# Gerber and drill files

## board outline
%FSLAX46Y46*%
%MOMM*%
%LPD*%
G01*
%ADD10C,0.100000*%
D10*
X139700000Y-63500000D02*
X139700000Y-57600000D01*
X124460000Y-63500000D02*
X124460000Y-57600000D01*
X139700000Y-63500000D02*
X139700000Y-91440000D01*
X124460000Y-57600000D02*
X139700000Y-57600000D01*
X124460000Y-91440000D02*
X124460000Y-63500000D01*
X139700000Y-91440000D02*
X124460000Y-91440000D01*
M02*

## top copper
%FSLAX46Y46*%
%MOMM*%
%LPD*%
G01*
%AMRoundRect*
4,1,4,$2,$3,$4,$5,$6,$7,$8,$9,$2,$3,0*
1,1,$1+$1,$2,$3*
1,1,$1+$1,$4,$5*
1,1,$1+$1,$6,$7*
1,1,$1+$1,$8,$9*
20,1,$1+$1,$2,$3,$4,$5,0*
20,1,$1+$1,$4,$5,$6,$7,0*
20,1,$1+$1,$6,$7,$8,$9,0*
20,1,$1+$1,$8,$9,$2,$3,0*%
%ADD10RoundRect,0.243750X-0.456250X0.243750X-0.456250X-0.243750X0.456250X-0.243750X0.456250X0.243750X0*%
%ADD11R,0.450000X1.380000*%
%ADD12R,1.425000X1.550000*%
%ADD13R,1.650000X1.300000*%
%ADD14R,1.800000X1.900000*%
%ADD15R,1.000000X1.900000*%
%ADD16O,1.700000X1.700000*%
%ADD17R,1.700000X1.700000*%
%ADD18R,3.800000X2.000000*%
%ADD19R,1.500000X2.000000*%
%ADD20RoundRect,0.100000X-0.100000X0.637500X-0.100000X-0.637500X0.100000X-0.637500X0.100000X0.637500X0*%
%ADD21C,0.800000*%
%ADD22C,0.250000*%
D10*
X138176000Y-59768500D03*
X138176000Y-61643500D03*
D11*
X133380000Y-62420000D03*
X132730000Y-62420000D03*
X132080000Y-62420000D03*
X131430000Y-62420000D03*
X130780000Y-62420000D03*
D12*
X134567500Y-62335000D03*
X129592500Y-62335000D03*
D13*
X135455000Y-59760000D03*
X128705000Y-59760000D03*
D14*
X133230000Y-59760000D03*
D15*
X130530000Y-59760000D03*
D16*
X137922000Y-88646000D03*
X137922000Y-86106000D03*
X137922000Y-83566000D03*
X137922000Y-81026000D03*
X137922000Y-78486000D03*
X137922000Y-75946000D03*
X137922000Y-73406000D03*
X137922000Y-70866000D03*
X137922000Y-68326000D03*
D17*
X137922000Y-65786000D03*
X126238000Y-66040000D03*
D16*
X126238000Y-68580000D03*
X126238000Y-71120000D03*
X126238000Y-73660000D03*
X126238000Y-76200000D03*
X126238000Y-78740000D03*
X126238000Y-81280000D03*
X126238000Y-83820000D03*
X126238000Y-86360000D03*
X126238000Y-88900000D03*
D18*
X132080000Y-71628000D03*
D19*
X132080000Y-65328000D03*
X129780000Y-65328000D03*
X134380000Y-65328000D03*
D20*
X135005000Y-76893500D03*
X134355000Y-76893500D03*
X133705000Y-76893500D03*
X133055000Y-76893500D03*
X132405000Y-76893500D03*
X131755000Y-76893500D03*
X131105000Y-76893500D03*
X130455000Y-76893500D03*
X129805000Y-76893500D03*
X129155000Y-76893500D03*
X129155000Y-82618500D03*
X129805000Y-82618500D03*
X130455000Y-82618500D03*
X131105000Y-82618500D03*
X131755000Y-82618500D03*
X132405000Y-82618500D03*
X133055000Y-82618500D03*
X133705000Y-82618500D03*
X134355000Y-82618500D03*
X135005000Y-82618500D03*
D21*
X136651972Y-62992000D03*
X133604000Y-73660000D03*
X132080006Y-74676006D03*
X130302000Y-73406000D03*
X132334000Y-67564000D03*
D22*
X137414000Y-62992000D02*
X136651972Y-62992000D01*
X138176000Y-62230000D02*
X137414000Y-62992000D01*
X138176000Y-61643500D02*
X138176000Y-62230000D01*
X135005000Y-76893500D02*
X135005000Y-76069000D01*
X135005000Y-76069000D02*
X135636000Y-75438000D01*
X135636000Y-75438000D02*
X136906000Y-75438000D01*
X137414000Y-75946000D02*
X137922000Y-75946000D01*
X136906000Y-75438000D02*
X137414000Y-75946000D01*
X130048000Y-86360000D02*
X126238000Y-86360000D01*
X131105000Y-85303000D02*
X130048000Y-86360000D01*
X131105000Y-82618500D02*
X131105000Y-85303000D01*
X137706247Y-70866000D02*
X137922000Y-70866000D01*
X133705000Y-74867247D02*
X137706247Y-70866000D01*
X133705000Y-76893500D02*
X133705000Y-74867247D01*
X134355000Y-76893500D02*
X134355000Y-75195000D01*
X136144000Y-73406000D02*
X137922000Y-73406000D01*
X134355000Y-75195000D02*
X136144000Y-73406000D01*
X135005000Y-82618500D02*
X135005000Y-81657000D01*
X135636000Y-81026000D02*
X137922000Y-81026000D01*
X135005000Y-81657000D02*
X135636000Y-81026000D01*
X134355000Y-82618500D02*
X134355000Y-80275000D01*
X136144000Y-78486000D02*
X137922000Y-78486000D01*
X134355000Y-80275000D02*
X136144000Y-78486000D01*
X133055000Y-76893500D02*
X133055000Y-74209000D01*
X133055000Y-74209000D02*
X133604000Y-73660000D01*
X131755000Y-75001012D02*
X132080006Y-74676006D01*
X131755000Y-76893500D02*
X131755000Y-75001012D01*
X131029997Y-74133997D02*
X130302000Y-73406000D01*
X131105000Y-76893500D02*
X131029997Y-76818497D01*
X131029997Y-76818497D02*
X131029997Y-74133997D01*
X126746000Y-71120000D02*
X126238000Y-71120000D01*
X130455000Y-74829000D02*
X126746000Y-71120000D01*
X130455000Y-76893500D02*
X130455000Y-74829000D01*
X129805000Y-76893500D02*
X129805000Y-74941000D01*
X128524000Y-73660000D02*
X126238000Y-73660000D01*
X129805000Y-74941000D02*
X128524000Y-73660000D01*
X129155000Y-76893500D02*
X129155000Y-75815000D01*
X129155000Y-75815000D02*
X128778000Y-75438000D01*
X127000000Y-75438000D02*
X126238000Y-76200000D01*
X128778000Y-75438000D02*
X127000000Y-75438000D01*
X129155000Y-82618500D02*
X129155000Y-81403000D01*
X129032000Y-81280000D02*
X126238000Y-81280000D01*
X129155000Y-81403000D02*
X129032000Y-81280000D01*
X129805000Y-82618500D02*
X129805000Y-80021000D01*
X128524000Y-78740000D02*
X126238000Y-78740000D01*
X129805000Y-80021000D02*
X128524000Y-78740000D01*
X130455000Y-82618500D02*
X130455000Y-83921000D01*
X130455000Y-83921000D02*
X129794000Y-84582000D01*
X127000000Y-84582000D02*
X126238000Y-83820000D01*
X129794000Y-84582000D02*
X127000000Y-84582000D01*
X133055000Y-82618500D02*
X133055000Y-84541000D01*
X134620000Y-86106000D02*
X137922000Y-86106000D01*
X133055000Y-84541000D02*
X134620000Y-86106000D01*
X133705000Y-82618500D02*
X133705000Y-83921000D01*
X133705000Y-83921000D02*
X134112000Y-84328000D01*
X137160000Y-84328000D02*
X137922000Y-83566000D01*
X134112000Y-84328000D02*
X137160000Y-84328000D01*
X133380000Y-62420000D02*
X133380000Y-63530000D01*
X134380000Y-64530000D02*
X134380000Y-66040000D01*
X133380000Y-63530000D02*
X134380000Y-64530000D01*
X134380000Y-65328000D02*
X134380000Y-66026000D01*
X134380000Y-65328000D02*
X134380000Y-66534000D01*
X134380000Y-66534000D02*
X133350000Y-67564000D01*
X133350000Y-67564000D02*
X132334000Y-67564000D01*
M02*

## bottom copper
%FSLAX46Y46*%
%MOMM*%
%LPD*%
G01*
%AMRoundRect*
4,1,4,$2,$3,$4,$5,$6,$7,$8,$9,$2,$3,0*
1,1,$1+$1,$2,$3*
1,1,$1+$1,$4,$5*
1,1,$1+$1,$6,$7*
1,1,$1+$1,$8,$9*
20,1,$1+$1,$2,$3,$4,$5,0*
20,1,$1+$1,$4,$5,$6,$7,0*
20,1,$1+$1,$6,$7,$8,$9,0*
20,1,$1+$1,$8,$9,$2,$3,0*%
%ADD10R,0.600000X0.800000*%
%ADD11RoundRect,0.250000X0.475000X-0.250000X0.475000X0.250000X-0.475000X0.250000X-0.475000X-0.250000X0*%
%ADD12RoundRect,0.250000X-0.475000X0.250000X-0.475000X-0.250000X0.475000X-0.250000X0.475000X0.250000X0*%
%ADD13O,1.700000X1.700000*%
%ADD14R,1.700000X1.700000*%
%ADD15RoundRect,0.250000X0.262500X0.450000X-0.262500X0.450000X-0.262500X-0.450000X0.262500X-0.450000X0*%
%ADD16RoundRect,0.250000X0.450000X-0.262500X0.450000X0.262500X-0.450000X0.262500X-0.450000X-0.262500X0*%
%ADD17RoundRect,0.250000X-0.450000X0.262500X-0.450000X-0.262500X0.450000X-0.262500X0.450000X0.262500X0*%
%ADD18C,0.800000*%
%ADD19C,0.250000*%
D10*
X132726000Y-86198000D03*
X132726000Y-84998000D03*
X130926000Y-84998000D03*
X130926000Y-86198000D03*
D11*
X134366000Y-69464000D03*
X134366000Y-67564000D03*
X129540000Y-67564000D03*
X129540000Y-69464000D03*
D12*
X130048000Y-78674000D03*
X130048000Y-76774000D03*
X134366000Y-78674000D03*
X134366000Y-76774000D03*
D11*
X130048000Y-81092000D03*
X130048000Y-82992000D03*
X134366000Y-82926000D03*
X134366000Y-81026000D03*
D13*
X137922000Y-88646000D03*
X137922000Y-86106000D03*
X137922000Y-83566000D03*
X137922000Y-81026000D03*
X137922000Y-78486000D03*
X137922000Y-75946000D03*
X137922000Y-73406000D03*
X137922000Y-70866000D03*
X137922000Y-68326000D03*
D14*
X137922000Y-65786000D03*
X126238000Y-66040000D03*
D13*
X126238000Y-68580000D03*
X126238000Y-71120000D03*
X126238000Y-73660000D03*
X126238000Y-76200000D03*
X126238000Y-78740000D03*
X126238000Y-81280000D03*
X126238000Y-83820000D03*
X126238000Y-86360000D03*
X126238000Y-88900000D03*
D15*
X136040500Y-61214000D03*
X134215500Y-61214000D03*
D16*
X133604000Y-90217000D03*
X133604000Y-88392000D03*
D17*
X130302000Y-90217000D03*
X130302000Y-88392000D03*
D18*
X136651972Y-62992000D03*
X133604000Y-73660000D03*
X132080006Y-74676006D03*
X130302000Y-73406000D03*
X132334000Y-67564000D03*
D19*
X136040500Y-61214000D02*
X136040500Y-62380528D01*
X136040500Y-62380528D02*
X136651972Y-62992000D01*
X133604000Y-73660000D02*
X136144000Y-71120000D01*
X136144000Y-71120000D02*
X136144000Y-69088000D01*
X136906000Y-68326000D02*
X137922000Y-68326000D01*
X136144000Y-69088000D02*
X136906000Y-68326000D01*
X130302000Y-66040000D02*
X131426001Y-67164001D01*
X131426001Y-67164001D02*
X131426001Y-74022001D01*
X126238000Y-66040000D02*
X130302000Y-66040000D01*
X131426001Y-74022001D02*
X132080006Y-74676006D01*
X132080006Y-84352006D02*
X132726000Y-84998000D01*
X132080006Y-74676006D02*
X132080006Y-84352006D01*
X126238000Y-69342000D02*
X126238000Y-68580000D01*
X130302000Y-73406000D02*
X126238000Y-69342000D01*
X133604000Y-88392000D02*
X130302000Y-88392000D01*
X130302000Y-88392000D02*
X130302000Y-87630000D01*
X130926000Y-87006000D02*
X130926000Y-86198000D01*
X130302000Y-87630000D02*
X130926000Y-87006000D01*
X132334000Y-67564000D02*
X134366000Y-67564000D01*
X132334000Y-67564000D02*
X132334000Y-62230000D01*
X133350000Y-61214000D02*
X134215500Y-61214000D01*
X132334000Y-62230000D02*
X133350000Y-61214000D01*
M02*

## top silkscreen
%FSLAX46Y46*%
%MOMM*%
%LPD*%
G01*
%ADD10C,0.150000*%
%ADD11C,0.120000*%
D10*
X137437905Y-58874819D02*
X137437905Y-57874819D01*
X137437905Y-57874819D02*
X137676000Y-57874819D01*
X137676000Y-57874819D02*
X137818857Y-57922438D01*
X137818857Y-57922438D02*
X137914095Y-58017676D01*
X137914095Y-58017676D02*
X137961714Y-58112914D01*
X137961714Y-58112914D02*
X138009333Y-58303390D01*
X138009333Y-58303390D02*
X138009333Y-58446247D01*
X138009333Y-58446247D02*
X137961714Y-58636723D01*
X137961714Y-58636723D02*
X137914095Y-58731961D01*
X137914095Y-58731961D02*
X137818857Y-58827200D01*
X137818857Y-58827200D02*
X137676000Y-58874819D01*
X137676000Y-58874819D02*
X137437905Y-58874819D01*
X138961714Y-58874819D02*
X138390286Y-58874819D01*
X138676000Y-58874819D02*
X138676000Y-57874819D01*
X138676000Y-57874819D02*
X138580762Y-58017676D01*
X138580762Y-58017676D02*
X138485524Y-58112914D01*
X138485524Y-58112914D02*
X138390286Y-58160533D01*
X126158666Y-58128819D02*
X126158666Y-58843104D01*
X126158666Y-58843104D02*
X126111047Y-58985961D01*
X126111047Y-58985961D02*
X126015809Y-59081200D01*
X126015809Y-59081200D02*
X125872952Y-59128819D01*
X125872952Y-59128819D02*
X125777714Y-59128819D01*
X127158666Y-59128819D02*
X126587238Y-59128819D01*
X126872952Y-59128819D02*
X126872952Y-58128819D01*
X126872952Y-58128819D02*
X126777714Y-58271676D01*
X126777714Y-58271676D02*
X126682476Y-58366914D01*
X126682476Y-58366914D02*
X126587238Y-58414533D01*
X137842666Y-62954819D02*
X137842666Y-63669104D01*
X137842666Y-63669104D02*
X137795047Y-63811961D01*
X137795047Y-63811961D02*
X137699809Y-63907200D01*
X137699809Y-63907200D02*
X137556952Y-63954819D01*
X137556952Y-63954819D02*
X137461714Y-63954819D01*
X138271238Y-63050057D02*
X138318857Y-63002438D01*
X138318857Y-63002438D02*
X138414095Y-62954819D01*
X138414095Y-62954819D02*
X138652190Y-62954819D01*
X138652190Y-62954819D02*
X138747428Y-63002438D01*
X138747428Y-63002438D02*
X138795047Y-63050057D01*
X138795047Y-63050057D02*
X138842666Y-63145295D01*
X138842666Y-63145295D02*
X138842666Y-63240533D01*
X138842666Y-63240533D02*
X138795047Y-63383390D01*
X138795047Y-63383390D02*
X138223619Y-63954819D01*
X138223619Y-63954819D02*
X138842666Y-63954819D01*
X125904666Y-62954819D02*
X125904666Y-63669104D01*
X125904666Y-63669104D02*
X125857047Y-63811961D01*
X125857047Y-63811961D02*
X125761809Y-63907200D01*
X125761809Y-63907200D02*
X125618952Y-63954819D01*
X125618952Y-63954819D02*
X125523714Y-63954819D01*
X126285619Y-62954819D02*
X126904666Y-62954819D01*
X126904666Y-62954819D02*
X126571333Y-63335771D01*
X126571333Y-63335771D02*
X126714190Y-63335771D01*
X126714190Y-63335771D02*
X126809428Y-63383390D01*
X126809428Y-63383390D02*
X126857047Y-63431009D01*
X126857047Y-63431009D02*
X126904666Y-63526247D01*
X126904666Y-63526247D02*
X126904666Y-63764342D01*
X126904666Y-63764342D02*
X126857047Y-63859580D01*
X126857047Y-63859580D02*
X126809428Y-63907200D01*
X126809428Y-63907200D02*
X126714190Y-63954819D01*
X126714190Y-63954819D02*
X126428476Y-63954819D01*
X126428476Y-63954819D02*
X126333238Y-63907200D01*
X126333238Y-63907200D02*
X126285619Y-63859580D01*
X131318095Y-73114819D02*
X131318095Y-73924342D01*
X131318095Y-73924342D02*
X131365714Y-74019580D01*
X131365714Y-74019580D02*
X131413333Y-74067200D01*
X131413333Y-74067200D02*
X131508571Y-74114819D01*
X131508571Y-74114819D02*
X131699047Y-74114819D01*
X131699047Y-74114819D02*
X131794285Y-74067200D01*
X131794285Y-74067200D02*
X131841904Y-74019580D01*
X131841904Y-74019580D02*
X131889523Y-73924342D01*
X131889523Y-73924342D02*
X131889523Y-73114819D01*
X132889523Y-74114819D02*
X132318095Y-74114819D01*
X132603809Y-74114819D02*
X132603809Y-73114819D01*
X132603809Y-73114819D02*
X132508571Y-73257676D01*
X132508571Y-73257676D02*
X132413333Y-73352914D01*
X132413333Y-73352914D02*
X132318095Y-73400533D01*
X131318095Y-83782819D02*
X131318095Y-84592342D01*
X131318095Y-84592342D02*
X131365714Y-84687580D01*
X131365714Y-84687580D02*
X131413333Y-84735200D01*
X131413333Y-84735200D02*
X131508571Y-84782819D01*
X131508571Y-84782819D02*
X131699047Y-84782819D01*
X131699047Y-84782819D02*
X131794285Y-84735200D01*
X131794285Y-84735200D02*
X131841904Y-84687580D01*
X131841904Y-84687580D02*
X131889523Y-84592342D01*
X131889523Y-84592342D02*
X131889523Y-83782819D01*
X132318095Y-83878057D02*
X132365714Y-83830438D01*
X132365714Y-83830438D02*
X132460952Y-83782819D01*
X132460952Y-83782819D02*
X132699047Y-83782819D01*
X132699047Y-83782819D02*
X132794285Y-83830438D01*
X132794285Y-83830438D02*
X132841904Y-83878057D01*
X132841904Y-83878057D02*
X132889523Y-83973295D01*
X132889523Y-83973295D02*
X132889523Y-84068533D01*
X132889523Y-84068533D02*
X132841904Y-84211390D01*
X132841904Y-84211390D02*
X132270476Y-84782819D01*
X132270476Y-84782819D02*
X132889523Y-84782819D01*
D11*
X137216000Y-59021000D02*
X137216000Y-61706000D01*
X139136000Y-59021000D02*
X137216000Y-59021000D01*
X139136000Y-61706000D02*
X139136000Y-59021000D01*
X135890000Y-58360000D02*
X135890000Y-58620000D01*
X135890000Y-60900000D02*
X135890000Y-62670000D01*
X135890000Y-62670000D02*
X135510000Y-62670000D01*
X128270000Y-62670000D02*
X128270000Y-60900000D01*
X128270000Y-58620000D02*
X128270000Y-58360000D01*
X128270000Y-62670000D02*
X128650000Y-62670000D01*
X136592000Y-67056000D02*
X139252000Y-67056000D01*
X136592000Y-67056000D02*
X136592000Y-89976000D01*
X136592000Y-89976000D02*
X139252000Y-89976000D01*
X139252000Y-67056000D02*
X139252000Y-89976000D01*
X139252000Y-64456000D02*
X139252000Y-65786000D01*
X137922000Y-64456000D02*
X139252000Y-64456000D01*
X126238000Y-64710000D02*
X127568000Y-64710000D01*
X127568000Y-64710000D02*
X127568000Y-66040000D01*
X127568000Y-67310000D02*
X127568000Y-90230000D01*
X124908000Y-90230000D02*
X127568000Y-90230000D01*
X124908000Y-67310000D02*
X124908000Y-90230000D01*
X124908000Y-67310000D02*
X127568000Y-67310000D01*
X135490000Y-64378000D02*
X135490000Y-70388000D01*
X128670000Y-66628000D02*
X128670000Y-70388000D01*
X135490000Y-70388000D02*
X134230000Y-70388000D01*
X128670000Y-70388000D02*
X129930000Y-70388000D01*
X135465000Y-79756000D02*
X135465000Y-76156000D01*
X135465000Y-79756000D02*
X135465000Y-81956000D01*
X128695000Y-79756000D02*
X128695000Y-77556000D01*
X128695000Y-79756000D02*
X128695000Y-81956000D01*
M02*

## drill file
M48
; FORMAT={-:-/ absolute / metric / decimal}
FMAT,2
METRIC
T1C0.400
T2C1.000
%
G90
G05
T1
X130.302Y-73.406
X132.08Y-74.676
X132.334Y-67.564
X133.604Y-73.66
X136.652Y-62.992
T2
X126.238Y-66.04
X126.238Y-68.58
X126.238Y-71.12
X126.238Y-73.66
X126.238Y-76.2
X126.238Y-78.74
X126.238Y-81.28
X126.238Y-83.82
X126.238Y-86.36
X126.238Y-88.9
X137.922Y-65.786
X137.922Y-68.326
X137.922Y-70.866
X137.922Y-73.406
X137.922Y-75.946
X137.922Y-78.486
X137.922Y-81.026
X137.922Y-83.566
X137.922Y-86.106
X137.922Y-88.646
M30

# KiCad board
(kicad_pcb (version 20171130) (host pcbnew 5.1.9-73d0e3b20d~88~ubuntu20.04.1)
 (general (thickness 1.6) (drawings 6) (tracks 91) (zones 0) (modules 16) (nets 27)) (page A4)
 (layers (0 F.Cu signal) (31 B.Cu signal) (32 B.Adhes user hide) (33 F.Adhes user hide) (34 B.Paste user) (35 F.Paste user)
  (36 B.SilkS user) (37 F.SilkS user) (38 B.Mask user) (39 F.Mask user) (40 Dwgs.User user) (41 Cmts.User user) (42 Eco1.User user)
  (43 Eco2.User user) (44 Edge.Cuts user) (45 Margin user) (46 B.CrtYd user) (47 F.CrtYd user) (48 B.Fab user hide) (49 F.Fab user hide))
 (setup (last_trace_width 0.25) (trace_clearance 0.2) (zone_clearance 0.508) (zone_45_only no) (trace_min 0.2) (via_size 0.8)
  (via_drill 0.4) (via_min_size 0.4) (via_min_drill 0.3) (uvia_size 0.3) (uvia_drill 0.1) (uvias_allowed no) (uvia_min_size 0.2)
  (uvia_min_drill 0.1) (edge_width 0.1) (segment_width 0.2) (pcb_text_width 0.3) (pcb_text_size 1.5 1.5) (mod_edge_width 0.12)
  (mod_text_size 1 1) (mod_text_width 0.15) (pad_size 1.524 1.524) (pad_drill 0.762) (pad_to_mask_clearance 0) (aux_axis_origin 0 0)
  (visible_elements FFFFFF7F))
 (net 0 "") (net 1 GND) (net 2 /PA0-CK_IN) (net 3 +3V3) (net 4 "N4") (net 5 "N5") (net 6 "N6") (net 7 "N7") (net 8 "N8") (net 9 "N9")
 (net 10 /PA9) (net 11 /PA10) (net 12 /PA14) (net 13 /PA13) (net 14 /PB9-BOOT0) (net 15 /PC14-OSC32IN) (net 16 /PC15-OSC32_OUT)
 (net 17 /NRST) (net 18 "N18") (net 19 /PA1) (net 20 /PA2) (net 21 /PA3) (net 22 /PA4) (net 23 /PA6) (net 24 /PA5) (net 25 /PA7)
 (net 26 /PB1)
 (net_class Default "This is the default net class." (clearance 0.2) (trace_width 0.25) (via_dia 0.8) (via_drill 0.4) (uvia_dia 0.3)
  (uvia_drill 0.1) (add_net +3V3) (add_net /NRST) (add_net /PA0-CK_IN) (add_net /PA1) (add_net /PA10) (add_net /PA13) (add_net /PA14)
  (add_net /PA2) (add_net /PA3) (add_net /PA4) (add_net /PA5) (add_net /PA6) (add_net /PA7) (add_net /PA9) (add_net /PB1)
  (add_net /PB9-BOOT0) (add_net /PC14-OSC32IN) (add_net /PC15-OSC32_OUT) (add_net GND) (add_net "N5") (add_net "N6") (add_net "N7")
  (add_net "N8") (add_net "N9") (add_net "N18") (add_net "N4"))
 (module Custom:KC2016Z (layer B.Cu) (at 131.826 85.598 180)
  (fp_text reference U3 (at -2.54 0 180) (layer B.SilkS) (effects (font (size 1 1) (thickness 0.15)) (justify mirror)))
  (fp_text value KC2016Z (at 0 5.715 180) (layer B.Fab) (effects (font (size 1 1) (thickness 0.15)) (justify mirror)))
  (pad 2 smd rect (at -0.9 -0.6 180) (size 0.6 0.8) (layers B.Cu B.Paste B.Mask) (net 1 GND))
  (pad 3 smd rect (at -0.9 0.6 180) (size 0.6 0.8) (layers B.Cu B.Paste B.Mask) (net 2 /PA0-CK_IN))
  (pad 4 smd rect (at 0.9 0.6 180) (size 0.6 0.8) (layers B.Cu B.Paste B.Mask) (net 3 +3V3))
  (pad 1 smd rect (at 0.9 -0.6 180) (size 0.6 0.8) (layers B.Cu B.Paste B.Mask) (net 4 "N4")))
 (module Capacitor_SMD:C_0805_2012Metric (layer B.Cu) (at 134.366 68.514 90)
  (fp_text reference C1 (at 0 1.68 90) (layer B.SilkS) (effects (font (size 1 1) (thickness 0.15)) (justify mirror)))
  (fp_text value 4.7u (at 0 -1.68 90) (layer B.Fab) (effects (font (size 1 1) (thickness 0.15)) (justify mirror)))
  (pad 1 smd roundrect (at -0.95 0 90) (size 1 1.45) (layers B.Cu B.Paste B.Mask) (roundrect_rratio 0.25) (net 1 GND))
  (pad 2 smd roundrect (at 0.95 0 90) (size 1 1.45) (layers B.Cu B.Paste B.Mask) (roundrect_rratio 0.25) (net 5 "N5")))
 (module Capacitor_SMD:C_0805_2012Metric (layer B.Cu) (at 129.54 68.514 90)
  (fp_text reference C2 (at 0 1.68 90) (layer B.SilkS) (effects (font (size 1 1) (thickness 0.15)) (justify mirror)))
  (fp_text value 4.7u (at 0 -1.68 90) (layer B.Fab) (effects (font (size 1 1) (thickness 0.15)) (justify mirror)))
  (pad 2 smd roundrect (at 0.95 0 90) (size 1 1.45) (layers B.Cu B.Paste B.Mask) (roundrect_rratio 0.25) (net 3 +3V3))
  (pad 1 smd roundrect (at -0.95 0 90) (size 1 1.45) (layers B.Cu B.Paste B.Mask) (roundrect_rratio 0.25) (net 1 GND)))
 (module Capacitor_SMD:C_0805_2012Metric (layer B.Cu) (at 130.048 77.724 270)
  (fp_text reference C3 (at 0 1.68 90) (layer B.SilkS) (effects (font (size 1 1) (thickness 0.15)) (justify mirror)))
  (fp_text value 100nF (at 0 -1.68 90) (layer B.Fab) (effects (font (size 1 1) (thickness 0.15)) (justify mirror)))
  (pad 2 smd roundrect (at 0.95 0 270) (size 1 1.45) (layers B.Cu B.Paste B.Mask) (roundrect_rratio 0.25) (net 3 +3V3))
  (pad 1 smd roundrect (at -0.95 0 270) (size 1 1.45) (layers B.Cu B.Paste B.Mask) (roundrect_rratio 0.25) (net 1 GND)))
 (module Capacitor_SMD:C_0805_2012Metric (layer B.Cu) (at 134.366 77.724 270)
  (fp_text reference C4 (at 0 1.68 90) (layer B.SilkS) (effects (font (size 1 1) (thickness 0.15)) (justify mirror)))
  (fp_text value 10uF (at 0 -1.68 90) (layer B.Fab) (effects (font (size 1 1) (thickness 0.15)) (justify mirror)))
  (pad 2 smd roundrect (at 0.95 0 270) (size 1 1.45) (layers B.Cu B.Paste B.Mask) (roundrect_rratio 0.25) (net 3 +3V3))
  (pad 1 smd roundrect (at -0.95 0 270) (size 1 1.45) (layers B.Cu B.Paste B.Mask) (roundrect_rratio 0.25) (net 1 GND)))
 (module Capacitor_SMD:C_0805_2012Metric (layer B.Cu) (at 130.048 82.042 90)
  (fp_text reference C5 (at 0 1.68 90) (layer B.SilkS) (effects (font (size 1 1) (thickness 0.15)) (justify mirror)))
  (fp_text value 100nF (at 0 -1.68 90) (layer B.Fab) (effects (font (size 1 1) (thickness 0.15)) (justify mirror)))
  (pad 2 smd roundrect (at 0.95 0 90) (size 1 1.45) (layers B.Cu B.Paste B.Mask) (roundrect_rratio 0.25) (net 3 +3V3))
  (pad 1 smd roundrect (at -0.95 0 90) (size 1 1.45) (layers B.Cu B.Paste B.Mask) (roundrect_rratio 0.25) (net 1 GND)))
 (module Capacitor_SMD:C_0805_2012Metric (layer B.Cu) (at 134.366 81.976 90)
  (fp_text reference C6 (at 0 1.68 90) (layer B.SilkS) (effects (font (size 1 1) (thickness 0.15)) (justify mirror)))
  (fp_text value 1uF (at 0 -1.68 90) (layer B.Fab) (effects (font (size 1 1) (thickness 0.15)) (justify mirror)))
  (pad 1 smd roundrect (at -0.95 0 90) (size 1 1.45) (layers B.Cu B.Paste B.Mask) (roundrect_rratio 0.25) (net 1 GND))
  (pad 2 smd roundrect (at 0.95 0 90) (size 1 1.45) (layers B.Cu B.Paste B.Mask) (roundrect_rratio 0.25) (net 3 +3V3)))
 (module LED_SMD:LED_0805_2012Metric (layer F.Cu) (at 138.176 60.706 270)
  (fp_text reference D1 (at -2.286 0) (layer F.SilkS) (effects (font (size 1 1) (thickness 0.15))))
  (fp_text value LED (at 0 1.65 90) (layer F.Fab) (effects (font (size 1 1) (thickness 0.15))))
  (fp_line (start -1.685 0.96) (end 1 0.96) (layer F.SilkS) (width 0.12))
  (fp_line (start -1.685 -0.96) (end -1.685 0.96) (layer F.SilkS) (width 0.12))
  (fp_line (start 1 -0.96) (end -1.685 -0.96) (layer F.SilkS) (width 0.12))
  (pad 1 smd roundrect (at -0.9375 0 270) (size 0.975 1.4) (layers F.Cu F.Paste F.Mask) (roundrect_rratio 0.25) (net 1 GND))
  (pad 2 smd roundrect (at 0.9375 0 270) (size 0.975 1.4) (layers F.Cu F.Paste F.Mask) (roundrect_rratio 0.25) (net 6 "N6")))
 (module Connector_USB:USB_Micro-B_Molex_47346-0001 (layer F.Cu) (at 132.08 60.96 180)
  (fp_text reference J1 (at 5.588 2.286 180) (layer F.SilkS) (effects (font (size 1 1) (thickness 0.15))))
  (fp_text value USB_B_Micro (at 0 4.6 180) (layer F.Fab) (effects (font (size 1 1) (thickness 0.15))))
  (fp_line (start -3.81 2.6) (end -3.81 2.34) (layer F.SilkS) (width 0.12))
  (fp_line (start -3.81 0.06) (end -3.81 -1.71) (layer F.SilkS) (width 0.12))
  (fp_line (start -3.81 -1.71) (end -3.43 -1.71) (layer F.SilkS) (width 0.12))
  (fp_line (start 3.81 -1.71) (end 3.81 0.06) (layer F.SilkS) (width 0.12))
  (fp_line (start 3.81 2.34) (end 3.81 2.6) (layer F.SilkS) (width 0.12))
  (fp_line (start 3.81 -1.71) (end 3.43 -1.71) (layer F.SilkS) (width 0.12))
  (pad 1 smd rect (at -1.3 -1.46 180) (size 0.45 1.38) (layers F.Cu F.Paste F.Mask) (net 5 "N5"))
  (pad 2 smd rect (at -0.65 -1.46 180) (size 0.45 1.38) (layers F.Cu F.Paste F.Mask) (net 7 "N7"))
  (pad 3 smd rect (at 0 -1.46 180) (size 0.45 1.38) (layers F.Cu F.Paste F.Mask) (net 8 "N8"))
  (pad 4 smd rect (at 0.65 -1.46 180) (size 0.45 1.38) (layers F.Cu F.Paste F.Mask) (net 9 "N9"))
  (pad 5 smd rect (at 1.3 -1.46 180) (size 0.45 1.38) (layers F.Cu F.Paste F.Mask) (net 1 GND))
  (pad 6 smd rect (at -2.4875 -1.375 180) (size 1.425 1.55) (layers F.Cu F.Paste F.Mask) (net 1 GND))
  (pad 6 smd rect (at 2.4875 -1.375 180) (size 1.425 1.55) (layers F.Cu F.Paste F.Mask) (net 1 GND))
  (pad 6 smd rect (at -3.375 1.2 180) (size 1.65 1.3) (layers F.Cu F.Paste F.Mask) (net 1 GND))
  (pad 6 smd rect (at 3.375 1.2 180) (size 1.65 1.3) (layers F.Cu F.Paste F.Mask) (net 1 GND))
  (pad 6 smd rect (at -1.15 1.2 180) (size 1.8 1.9) (layers F.Cu F.Paste F.Mask) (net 1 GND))
  (pad 6 smd rect (at 1.55 1.2 180) (size 1 1.9) (layers F.Cu F.Paste F.Mask) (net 1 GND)))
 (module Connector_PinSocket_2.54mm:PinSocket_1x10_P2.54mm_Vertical (layer F.Cu) (at 137.922 65.786)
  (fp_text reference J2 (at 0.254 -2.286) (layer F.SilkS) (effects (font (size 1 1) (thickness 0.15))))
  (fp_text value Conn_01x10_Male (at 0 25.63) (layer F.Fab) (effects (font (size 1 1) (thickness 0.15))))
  (fp_line (start -1.33 1.27) (end 1.33 1.27) (layer F.SilkS) (width 0.12))
  (fp_line (start -1.33 1.27) (end -1.33 24.19) (layer F.SilkS) (width 0.12))
  (fp_line (start -1.33 24.19) (end 1.33 24.19) (layer F.SilkS) (width 0.12))
  (fp_line (start 1.33 1.27) (end 1.33 24.19) (layer F.SilkS) (width 0.12))
  (fp_line (start 1.33 -1.33) (end 1.33 0) (layer F.SilkS) (width 0.12))
  (fp_line (start 0 -1.33) (end 1.33 -1.33) (layer F.SilkS) (width 0.12))
  (pad 10 thru_hole oval (at 0 22.86) (size 1.7 1.7) (drill 1) (layers *.Cu *.Mask) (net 3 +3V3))
  (pad 9 thru_hole oval (at 0 20.32) (size 1.7 1.7) (drill 1) (layers *.Cu *.Mask) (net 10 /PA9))
  (pad 8 thru_hole oval (at 0 17.78) (size 1.7 1.7) (drill 1) (layers *.Cu *.Mask) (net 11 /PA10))
  (pad 7 thru_hole oval (at 0 15.24) (size 1.7 1.7) (drill 1) (layers *.Cu *.Mask) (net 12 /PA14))
  (pad 6 thru_hole oval (at 0 12.7) (size 1.7 1.7) (drill 1) (layers *.Cu *.Mask) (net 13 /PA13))
  (pad 5 thru_hole oval (at 0 10.16) (size 1.7 1.7) (drill 1) (layers *.Cu *.Mask) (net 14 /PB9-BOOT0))
  (pad 4 thru_hole oval (at 0 7.62) (size 1.7 1.7) (drill 1) (layers *.Cu *.Mask) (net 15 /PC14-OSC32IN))
  (pad 3 thru_hole oval (at 0 5.08) (size 1.7 1.7) (drill 1) (layers *.Cu *.Mask) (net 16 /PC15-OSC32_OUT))
  (pad 2 thru_hole oval (at 0 2.54) (size 1.7 1.7) (drill 1) (layers *.Cu *.Mask) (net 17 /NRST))
  (pad 1 thru_hole rect (at 0 0) (size 1.7 1.7) (drill 1) (layers *.Cu *.Mask) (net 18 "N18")))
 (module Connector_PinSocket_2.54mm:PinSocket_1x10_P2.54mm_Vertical (layer F.Cu) (at 126.238 66.04)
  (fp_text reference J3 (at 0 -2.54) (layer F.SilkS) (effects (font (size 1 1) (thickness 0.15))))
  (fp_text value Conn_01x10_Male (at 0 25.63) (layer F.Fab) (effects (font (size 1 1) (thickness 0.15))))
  (fp_line (start 0 -1.33) (end 1.33 -1.33) (layer F.SilkS) (width 0.12))
  (fp_line (start 1.33 -1.33) (end 1.33 0) (layer F.SilkS) (width 0.12))
  (fp_line (start 1.33 1.27) (end 1.33 24.19) (layer F.SilkS) (width 0.12))
  (fp_line (start -1.33 24.19) (end 1.33 24.19) (layer F.SilkS) (width 0.12))
  (fp_line (start -1.33 1.27) (end -1.33 24.19) (layer F.SilkS) (width 0.12))
  (fp_line (start -1.33 1.27) (end 1.33 1.27) (layer F.SilkS) (width 0.12))
  (pad 1 thru_hole rect (at 0 0) (size 1.7 1.7) (drill 1) (layers *.Cu *.Mask) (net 2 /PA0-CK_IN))
  (pad 2 thru_hole oval (at 0 2.54) (size 1.7 1.7) (drill 1) (layers *.Cu *.Mask) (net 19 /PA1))
  (pad 3 thru_hole oval (at 0 5.08) (size 1.7 1.7) (drill 1) (layers *.Cu *.Mask) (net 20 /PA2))
  (pad 4 thru_hole oval (at 0 7.62) (size 1.7 1.7) (drill 1) (layers *.Cu *.Mask) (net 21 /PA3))
  (pad 5 thru_hole oval (at 0 10.16) (size 1.7 1.7) (drill 1) (layers *.Cu *.Mask) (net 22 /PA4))
  (pad 6 thru_hole oval (at 0 12.7) (size 1.7 1.7) (drill 1) (layers *.Cu *.Mask) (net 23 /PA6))
  (pad 7 thru_hole oval (at 0 15.24) (size 1.7 1.7) (drill 1) (layers *.Cu *.Mask) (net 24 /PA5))
  (pad 8 thru_hole oval (at 0 17.78) (size 1.7 1.7) (drill 1) (layers *.Cu *.Mask) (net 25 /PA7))
  (pad 9 thru_hole oval (at 0 20.32) (size 1.7 1.7) (drill 1) (layers *.Cu *.Mask) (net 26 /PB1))
  (pad 10 thru_hole oval (at 0 22.86) (size 1.7 1.7) (drill 1) (layers *.Cu *.Mask) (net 1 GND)))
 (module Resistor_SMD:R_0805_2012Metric (layer B.Cu) (at 135.128 61.214 180)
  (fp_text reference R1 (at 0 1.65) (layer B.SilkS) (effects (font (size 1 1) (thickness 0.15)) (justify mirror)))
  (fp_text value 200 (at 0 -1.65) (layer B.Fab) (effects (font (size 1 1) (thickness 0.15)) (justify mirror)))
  (pad 1 smd roundrect (at -0.9125 0 180) (size 1.025 1.4) (layers B.Cu B.Paste B.Mask) (roundrect_rratio 0.243902) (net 6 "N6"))
  (pad 2 smd roundrect (at 0.9125 0 180) (size 1.025 1.4) (layers B.Cu B.Paste B.Mask) (roundrect_rratio 0.243902) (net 5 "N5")))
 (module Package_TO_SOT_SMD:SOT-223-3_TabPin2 (layer F.Cu) (at 132.08 68.478 270)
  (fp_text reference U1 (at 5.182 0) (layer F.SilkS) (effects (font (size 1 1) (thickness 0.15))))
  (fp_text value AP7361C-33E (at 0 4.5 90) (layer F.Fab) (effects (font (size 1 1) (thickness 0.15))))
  (fp_line (start -4.1 -3.41) (end 1.91 -3.41) (layer F.SilkS) (width 0.12))
  (fp_line (start -1.85 3.41) (end 1.91 3.41) (layer F.SilkS) (width 0.12))
  (fp_line (start 1.91 -3.41) (end 1.91 -2.15) (layer F.SilkS) (width 0.12))
  (fp_line (start 1.91 3.41) (end 1.91 2.15) (layer F.SilkS) (width 0.12))
  (pad 2 smd rect (at 3.15 0 270) (size 2 3.8) (layers F.Cu F.Paste F.Mask) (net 1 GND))
  (pad 2 smd rect (at -3.15 0 270) (size 2 1.5) (layers F.Cu F.Paste F.Mask) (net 1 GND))
  (pad 3 smd rect (at -3.15 2.3 270) (size 2 1.5) (layers F.Cu F.Paste F.Mask) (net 3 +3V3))
  (pad 1 smd rect (at -3.15 -2.3 270) (size 2 1.5) (layers F.Cu F.Paste F.Mask) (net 5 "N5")))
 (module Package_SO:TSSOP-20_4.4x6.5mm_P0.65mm (layer F.Cu) (at 132.08 79.756 270)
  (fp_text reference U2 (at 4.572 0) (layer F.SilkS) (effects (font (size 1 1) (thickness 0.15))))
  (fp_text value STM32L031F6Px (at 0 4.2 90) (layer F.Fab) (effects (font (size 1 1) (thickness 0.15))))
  (fp_line (start 0 -3.385) (end -3.6 -3.385) (layer F.SilkS) (width 0.12))
  (fp_line (start 0 -3.385) (end 2.2 -3.385) (layer F.SilkS) (width 0.12))
  (fp_line (start 0 3.385) (end -2.2 3.385) (layer F.SilkS) (width 0.12))
  (fp_line (start 0 3.385) (end 2.2 3.385) (layer F.SilkS) (width 0.12))
  (pad 1 smd roundrect (at -2.8625 -2.925 270) (size 1.475 0.4) (layers F.Cu F.Paste F.Mask) (roundrect_rratio 0.25) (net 14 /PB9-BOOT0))
  (pad 2 smd roundrect (at -2.8625 -2.275 270) (size 1.475 0.4) (layers F.Cu F.Paste F.Mask) (roundrect_rratio 0.25) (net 15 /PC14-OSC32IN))
  (pad 3 smd roundrect (at -2.8625 -1.625 270) (size 1.475 0.4) (layers F.Cu F.Paste F.Mask) (roundrect_rratio 0.25)
   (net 16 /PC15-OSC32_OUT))
  (pad 4 smd roundrect (at -2.8625 -0.975 270) (size 1.475 0.4) (layers F.Cu F.Paste F.Mask) (roundrect_rratio 0.25) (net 17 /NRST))
  (pad 5 smd roundrect (at -2.8625 -0.325 270) (size 1.475 0.4) (layers F.Cu F.Paste F.Mask) (roundrect_rratio 0.25) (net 3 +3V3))
  (pad 6 smd roundrect (at -2.8625 0.325 270) (size 1.475 0.4) (layers F.Cu F.Paste F.Mask) (roundrect_rratio 0.25) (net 2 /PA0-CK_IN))
  (pad 7 smd roundrect (at -2.8625 0.975 270) (size 1.475 0.4) (layers F.Cu F.Paste F.Mask) (roundrect_rratio 0.25) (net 19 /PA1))
  (pad 8 smd roundrect (at -2.8625 1.625 270) (size 1.475 0.4) (layers F.Cu F.Paste F.Mask) (roundrect_rratio 0.25) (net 20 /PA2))
  (pad 9 smd roundrect (at -2.8625 2.275 270) (size 1.475 0.4) (layers F.Cu F.Paste F.Mask) (roundrect_rratio 0.25) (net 21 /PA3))
  (pad 10 smd roundrect (at -2.8625 2.925 270) (size 1.475 0.4) (layers F.Cu F.Paste F.Mask) (roundrect_rratio 0.25) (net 22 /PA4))
  (pad 11 smd roundrect (at 2.8625 2.925 270) (size 1.475 0.4) (layers F.Cu F.Paste F.Mask) (roundrect_rratio 0.25) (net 24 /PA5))
  (pad 12 smd roundrect (at 2.8625 2.275 270) (size 1.475 0.4) (layers F.Cu F.Paste F.Mask) (roundrect_rratio 0.25) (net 23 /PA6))
  (pad 13 smd roundrect (at 2.8625 1.625 270) (size 1.475 0.4) (layers F.Cu F.Paste F.Mask) (roundrect_rratio 0.25) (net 25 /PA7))
  (pad 14 smd roundrect (at 2.8625 0.975 270) (size 1.475 0.4) (layers F.Cu F.Paste F.Mask) (roundrect_rratio 0.25) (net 26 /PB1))
  (pad 15 smd roundrect (at 2.8625 0.325 270) (size 1.475 0.4) (layers F.Cu F.Paste F.Mask) (roundrect_rratio 0.25) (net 1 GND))
  (pad 16 smd roundrect (at 2.8625 -0.325 270) (size 1.475 0.4) (layers F.Cu F.Paste F.Mask) (roundrect_rratio 0.25) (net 3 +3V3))
  (pad 17 smd roundrect (at 2.8625 -0.975 270) (size 1.475 0.4) (layers F.Cu F.Paste F.Mask) (roundrect_rratio 0.25) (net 10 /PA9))
  (pad 18 smd roundrect (at 2.8625 -1.625 270) (size 1.475 0.4) (layers F.Cu F.Paste F.Mask) (roundrect_rratio 0.25) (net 11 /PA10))
  (pad 19 smd roundrect (at 2.8625 -2.275 270) (size 1.475 0.4) (layers F.Cu F.Paste F.Mask) (roundrect_rratio 0.25) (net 13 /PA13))
  (pad 20 smd roundrect (at 2.8625 -2.925 270) (size 1.475 0.4) (layers F.Cu F.Paste F.Mask) (roundrect_rratio 0.25) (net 12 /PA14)))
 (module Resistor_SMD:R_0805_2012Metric (layer B.Cu) (at 133.604 89.3045 90)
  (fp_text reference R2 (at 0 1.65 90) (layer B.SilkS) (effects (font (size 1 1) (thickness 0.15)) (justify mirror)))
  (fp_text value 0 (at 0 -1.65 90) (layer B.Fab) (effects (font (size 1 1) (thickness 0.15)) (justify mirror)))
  (pad 1 smd roundrect (at -0.9125 0 90) (size 1.025 1.4) (layers B.Cu B.Paste B.Mask) (roundrect_rratio 0.243902) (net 3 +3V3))
  (pad 2 smd roundrect (at 0.9125 0 90) (size 1.025 1.4) (layers B.Cu B.Paste B.Mask) (roundrect_rratio 0.243902) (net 4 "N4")))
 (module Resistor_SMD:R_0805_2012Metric (layer B.Cu) (at 130.302 89.3045 270)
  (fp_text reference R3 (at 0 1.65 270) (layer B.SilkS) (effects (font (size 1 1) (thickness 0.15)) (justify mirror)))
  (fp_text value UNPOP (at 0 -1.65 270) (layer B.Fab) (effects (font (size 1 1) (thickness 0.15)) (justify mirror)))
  (pad 2 smd roundrect (at 0.9125 0 270) (size 1.025 1.4) (layers B.Cu B.Paste B.Mask) (roundrect_rratio 0.243902) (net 1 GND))
  (pad 1 smd roundrect (at -0.9125 0 270) (size 1.025 1.4) (layers B.Cu B.Paste B.Mask) (roundrect_rratio 0.243902) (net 4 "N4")))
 (gr_line (start 139.7 63.5) (end 139.7 57.6) (layer Edge.Cuts) (width 0.1))
 (gr_line (start 124.46 63.5) (end 124.46 57.6) (layer Edge.Cuts) (width 0.1))
 (gr_line (start 139.7 63.5) (end 139.7 91.44) (layer Edge.Cuts) (width 0.1))
 (gr_line (start 124.46 57.6) (end 139.7 57.6) (layer Edge.Cuts) (width 0.1))
 (gr_line (start 124.46 91.44) (end 124.46 63.5) (layer Edge.Cuts) (width 0.1))
 (gr_line (start 139.7 91.44) (end 124.46 91.44) (layer Edge.Cuts) (width 0.1))
 (via (at 136.651972 62.992) (size 0.8) (drill 0.4) (layers F.Cu B.Cu) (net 6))
 (segment (start 136.0405 61.214) (end 136.0405 62.380528) (width 0.25) (layer B.Cu) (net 6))
 (segment (start 136.0405 62.380528) (end 136.651972 62.992) (width 0.25) (layer B.Cu) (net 6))
 (segment (start 137.414 62.992) (end 136.651972 62.992) (width 0.25) (layer F.Cu) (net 6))
 (segment (start 138.176 62.23) (end 137.414 62.992) (width 0.25) (layer F.Cu) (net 6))
 (segment (start 138.176 61.6435) (end 138.176 62.23) (width 0.25) (layer F.Cu) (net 6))
 (segment (start 135.005 76.8935) (end 135.005 76.069) (width 0.25) (layer F.Cu) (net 14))
 (segment (start 135.005 76.069) (end 135.636 75.438) (width 0.25) (layer F.Cu) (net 14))
 (segment (start 135.636 75.438) (end 136.906 75.438) (width 0.25) (layer F.Cu) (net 14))
 (segment (start 137.414 75.946) (end 137.922 75.946) (width 0.25) (layer F.Cu) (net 14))
 (segment (start 136.906 75.438) (end 137.414 75.946) (width 0.25) (layer F.Cu) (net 14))
 (segment (start 130.048 86.36) (end 126.238 86.36) (width 0.25) (layer F.Cu) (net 26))
 (segment (start 131.105 85.303) (end 130.048 86.36) (width 0.25) (layer F.Cu) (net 26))
 (segment (start 131.105 82.6185) (end 131.105 85.303) (width 0.25) (layer F.Cu) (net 26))
 (segment (start 137.706247 70.866) (end 137.922 70.866) (width 0.25) (layer F.Cu) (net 16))
 (segment (start 133.705 74.867247) (end 137.706247 70.866) (width 0.25) (layer F.Cu) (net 16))
 (segment (start 133.705 76.8935) (end 133.705 74.867247) (width 0.25) (layer F.Cu) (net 16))
 (segment (start 134.355 76.8935) (end 134.355 75.195) (width 0.25) (layer F.Cu) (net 15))
 (segment (start 136.144 73.406) (end 137.922 73.406) (width 0.25) (layer F.Cu) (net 15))
 (segment (start 134.355 75.195) (end 136.144 73.406) (width 0.25) (layer F.Cu) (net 15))
 (segment (start 135.005 82.6185) (end 135.005 81.657) (width 0.25) (layer F.Cu) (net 12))
 (segment (start 135.636 81.026) (end 137.922 81.026) (width 0.25) (layer F.Cu) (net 12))
 (segment (start 135.005 81.657) (end 135.636 81.026) (width 0.25) (layer F.Cu) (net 12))
 (segment (start 134.355 82.6185) (end 134.355 80.275) (width 0.25) (layer F.Cu) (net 13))
 (segment (start 136.144 78.486) (end 137.922 78.486) (width 0.25) (layer F.Cu) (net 13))
 (segment (start 134.355 80.275) (end 136.144 78.486) (width 0.25) (layer F.Cu) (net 13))
 (segment (start 133.055 76.8935) (end 133.055 74.209) (width 0.25) (layer F.Cu) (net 17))
 (via (at 133.604 73.66) (size 0.8) (drill 0.4) (layers F.Cu B.Cu) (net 17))
 (segment (start 133.055 74.209) (end 133.604 73.66) (width 0.25) (layer F.Cu) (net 17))
 (segment (start 133.604 73.66) (end 136.144 71.12) (width 0.25) (layer B.Cu) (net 17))
 (segment (start 136.144 71.12) (end 136.144 69.088) (width 0.25) (layer B.Cu) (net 17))
 (segment (start 136.906 68.326) (end 137.922 68.326) (width 0.25) (layer B.Cu) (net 17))
 (segment (start 136.144 69.088) (end 136.906 68.326) (width 0.25) (layer B.Cu) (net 17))
 (via (at 132.080006 74.676006) (size 0.8) (drill 0.4) (layers F.Cu B.Cu) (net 2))
 (segment (start 130.302 66.04) (end 131.426001 67.164001) (width 0.25) (layer B.Cu) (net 2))
 (segment (start 131.426001 67.164001) (end 131.426001 74.022001) (width 0.25) (layer B.Cu) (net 2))
 (segment (start 131.755 75.001012) (end 132.080006 74.676006) (width 0.25) (layer F.Cu) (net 2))
 (segment (start 131.755 76.8935) (end 131.755 75.001012) (width 0.25) (layer F.Cu) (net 2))
 (segment (start 126.238 66.04) (end 130.302 66.04) (width 0.25) (layer B.Cu) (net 2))
 (segment (start 131.426001 74.022001) (end 132.080006 74.676006) (width 0.25) (layer B.Cu) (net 2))
 (segment (start 132.080006 84.352006) (end 132.726 84.998) (width 0.25) (layer B.Cu) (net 2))
 (segment (start 132.080006 74.676006) (end 132.080006 84.352006) (width 0.25) (layer B.Cu) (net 2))
 (via (at 130.302 73.406) (size 0.8) (drill 0.4) (layers F.Cu B.Cu) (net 19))
 (segment (start 126.238 69.342) (end 126.238 68.58) (width 0.25) (layer B.Cu) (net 19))
 (segment (start 130.302 73.406) (end 126.238 69.342) (width 0.25) (layer B.Cu) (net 19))
 (segment (start 131.029997 74.133997) (end 130.302 73.406) (width 0.25) (layer F.Cu) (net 19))
 (segment (start 131.105 76.8935) (end 131.029997 76.818497) (width 0.25) (layer F.Cu) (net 19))
 (segment (start 131.029997 76.818497) (end 131.029997 74.133997) (width 0.25) (layer F.Cu) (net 19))
 (segment (start 126.746 71.12) (end 126.238 71.12) (width 0.25) (layer F.Cu) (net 20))
 (segment (start 130.455 74.829) (end 126.746 71.12) (width 0.25) (layer F.Cu) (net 20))
 (segment (start 130.455 76.8935) (end 130.455 74.829) (width 0.25) (layer F.Cu) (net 20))
 (segment (start 129.805 76.8935) (end 129.805 74.941) (width 0.25) (layer F.Cu) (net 21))
 (segment (start 128.524 73.66) (end 126.238 73.66) (width 0.25) (layer F.Cu) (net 21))
 (segment (start 129.805 74.941) (end 128.524 73.66) (width 0.25) (layer F.Cu) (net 21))
 (segment (start 129.155 76.8935) (end 129.155 75.815) (width 0.25) (layer F.Cu) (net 22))
 (segment (start 129.155 75.815) (end 128.778 75.438) (width 0.25) (layer F.Cu) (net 22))
 (segment (start 127 75.438) (end 126.238 76.2) (width 0.25) (layer F.Cu) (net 22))
 (segment (start 128.778 75.438) (end 127 75.438) (width 0.25) (layer F.Cu) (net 22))
 (segment (start 129.155 82.6185) (end 129.155 81.403) (width 0.25) (layer F.Cu) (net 24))
 (segment (start 129.032 81.28) (end 126.238 81.28) (width 0.25) (layer F.Cu) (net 24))
 (segment (start 129.155 81.403) (end 129.032 81.28) (width 0.25) (layer F.Cu) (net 24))
 (segment (start 129.805 82.6185) (end 129.805 80.021) (width 0.25) (layer F.Cu) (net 23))
 (segment (start 128.524 78.74) (end 126.238 78.74) (width 0.25) (layer F.Cu) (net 23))
 (segment (start 129.805 80.021) (end 128.524 78.74) (width 0.25) (layer F.Cu) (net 23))
 (segment (start 130.455 82.6185) (end 130.455 83.921) (width 0.25) (layer F.Cu) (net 25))
 (segment (start 130.455 83.921) (end 129.794 84.582) (width 0.25) (layer F.Cu) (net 25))
 (segment (start 127 84.582) (end 126.238 83.82) (width 0.25) (layer F.Cu) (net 25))
 (segment (start 129.794 84.582) (end 127 84.582) (width 0.25) (layer F.Cu) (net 25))
 (segment (start 133.055 82.6185) (end 133.055 84.541) (width 0.25) (layer F.Cu) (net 10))
 (segment (start 134.62 86.106) (end 137.922 86.106) (width 0.25) (layer F.Cu) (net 10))
 (segment (start 133.055 84.541) (end 134.62 86.106) (width 0.25) (layer F.Cu) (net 10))
 (segment (start 133.705 82.6185) (end 133.705 83.921) (width 0.25) (layer F.Cu) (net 11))
 (segment (start 133.705 83.921) (end 134.112 84.328) (width 0.25) (layer F.Cu) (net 11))
 (segment (start 137.16 84.328) (end 137.922 83.566) (width 0.25) (layer F.Cu) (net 11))
 (segment (start 134.112 84.328) (end 137.16 84.328) (width 0.25) (layer F.Cu) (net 11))
 (segment (start 133.604 88.392) (end 130.302 88.392) (width 0.25) (layer B.Cu) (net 4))
 (segment (start 130.302 88.392) (end 130.302 87.63) (width 0.25) (layer B.Cu) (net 4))
 (segment (start 130.926 87.006) (end 130.926 86.198) (width 0.25) (layer B.Cu) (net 4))
 (segment (start 130.302 87.63) (end 130.926 87.006) (width 0.25) (layer B.Cu) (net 4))
 (segment (start 133.38 62.42) (end 133.38 63.53) (width 0.25) (layer F.Cu) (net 5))
 (segment (start 134.38 64.53) (end 134.38 66.04) (width 0.25) (layer F.Cu) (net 5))
 (segment (start 133.38 63.53) (end 134.38 64.53) (width 0.25) (layer F.Cu) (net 5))
 (segment (start 134.38 65.328) (end 134.38 66.026) (width 0.25) (layer F.Cu) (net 5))
 (segment (start 134.38 65.328) (end 134.38 66.534) (width 0.25) (layer F.Cu) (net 5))
 (segment (start 134.38 66.534) (end 133.35 67.564) (width 0.25) (layer F.Cu) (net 5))
 (via (at 132.334 67.564) (size 0.8) (drill 0.4) (layers F.Cu B.Cu) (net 5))
 (segment (start 133.35 67.564) (end 132.334 67.564) (width 0.25) (layer F.Cu) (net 5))
 (segment (start 132.334 67.564) (end 134.366 67.564) (width 0.25) (layer B.Cu) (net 5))
 (segment (start 132.334 67.564) (end 132.334 62.23) (width 0.25) (layer B.Cu) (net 5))
 (segment (start 133.35 61.214) (end 134.2155 61.214) (width 0.25) (layer B.Cu) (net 5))
 (segment (start 132.334 62.23) (end 133.35 61.214) (width 0.25) (layer B.Cu) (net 5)))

